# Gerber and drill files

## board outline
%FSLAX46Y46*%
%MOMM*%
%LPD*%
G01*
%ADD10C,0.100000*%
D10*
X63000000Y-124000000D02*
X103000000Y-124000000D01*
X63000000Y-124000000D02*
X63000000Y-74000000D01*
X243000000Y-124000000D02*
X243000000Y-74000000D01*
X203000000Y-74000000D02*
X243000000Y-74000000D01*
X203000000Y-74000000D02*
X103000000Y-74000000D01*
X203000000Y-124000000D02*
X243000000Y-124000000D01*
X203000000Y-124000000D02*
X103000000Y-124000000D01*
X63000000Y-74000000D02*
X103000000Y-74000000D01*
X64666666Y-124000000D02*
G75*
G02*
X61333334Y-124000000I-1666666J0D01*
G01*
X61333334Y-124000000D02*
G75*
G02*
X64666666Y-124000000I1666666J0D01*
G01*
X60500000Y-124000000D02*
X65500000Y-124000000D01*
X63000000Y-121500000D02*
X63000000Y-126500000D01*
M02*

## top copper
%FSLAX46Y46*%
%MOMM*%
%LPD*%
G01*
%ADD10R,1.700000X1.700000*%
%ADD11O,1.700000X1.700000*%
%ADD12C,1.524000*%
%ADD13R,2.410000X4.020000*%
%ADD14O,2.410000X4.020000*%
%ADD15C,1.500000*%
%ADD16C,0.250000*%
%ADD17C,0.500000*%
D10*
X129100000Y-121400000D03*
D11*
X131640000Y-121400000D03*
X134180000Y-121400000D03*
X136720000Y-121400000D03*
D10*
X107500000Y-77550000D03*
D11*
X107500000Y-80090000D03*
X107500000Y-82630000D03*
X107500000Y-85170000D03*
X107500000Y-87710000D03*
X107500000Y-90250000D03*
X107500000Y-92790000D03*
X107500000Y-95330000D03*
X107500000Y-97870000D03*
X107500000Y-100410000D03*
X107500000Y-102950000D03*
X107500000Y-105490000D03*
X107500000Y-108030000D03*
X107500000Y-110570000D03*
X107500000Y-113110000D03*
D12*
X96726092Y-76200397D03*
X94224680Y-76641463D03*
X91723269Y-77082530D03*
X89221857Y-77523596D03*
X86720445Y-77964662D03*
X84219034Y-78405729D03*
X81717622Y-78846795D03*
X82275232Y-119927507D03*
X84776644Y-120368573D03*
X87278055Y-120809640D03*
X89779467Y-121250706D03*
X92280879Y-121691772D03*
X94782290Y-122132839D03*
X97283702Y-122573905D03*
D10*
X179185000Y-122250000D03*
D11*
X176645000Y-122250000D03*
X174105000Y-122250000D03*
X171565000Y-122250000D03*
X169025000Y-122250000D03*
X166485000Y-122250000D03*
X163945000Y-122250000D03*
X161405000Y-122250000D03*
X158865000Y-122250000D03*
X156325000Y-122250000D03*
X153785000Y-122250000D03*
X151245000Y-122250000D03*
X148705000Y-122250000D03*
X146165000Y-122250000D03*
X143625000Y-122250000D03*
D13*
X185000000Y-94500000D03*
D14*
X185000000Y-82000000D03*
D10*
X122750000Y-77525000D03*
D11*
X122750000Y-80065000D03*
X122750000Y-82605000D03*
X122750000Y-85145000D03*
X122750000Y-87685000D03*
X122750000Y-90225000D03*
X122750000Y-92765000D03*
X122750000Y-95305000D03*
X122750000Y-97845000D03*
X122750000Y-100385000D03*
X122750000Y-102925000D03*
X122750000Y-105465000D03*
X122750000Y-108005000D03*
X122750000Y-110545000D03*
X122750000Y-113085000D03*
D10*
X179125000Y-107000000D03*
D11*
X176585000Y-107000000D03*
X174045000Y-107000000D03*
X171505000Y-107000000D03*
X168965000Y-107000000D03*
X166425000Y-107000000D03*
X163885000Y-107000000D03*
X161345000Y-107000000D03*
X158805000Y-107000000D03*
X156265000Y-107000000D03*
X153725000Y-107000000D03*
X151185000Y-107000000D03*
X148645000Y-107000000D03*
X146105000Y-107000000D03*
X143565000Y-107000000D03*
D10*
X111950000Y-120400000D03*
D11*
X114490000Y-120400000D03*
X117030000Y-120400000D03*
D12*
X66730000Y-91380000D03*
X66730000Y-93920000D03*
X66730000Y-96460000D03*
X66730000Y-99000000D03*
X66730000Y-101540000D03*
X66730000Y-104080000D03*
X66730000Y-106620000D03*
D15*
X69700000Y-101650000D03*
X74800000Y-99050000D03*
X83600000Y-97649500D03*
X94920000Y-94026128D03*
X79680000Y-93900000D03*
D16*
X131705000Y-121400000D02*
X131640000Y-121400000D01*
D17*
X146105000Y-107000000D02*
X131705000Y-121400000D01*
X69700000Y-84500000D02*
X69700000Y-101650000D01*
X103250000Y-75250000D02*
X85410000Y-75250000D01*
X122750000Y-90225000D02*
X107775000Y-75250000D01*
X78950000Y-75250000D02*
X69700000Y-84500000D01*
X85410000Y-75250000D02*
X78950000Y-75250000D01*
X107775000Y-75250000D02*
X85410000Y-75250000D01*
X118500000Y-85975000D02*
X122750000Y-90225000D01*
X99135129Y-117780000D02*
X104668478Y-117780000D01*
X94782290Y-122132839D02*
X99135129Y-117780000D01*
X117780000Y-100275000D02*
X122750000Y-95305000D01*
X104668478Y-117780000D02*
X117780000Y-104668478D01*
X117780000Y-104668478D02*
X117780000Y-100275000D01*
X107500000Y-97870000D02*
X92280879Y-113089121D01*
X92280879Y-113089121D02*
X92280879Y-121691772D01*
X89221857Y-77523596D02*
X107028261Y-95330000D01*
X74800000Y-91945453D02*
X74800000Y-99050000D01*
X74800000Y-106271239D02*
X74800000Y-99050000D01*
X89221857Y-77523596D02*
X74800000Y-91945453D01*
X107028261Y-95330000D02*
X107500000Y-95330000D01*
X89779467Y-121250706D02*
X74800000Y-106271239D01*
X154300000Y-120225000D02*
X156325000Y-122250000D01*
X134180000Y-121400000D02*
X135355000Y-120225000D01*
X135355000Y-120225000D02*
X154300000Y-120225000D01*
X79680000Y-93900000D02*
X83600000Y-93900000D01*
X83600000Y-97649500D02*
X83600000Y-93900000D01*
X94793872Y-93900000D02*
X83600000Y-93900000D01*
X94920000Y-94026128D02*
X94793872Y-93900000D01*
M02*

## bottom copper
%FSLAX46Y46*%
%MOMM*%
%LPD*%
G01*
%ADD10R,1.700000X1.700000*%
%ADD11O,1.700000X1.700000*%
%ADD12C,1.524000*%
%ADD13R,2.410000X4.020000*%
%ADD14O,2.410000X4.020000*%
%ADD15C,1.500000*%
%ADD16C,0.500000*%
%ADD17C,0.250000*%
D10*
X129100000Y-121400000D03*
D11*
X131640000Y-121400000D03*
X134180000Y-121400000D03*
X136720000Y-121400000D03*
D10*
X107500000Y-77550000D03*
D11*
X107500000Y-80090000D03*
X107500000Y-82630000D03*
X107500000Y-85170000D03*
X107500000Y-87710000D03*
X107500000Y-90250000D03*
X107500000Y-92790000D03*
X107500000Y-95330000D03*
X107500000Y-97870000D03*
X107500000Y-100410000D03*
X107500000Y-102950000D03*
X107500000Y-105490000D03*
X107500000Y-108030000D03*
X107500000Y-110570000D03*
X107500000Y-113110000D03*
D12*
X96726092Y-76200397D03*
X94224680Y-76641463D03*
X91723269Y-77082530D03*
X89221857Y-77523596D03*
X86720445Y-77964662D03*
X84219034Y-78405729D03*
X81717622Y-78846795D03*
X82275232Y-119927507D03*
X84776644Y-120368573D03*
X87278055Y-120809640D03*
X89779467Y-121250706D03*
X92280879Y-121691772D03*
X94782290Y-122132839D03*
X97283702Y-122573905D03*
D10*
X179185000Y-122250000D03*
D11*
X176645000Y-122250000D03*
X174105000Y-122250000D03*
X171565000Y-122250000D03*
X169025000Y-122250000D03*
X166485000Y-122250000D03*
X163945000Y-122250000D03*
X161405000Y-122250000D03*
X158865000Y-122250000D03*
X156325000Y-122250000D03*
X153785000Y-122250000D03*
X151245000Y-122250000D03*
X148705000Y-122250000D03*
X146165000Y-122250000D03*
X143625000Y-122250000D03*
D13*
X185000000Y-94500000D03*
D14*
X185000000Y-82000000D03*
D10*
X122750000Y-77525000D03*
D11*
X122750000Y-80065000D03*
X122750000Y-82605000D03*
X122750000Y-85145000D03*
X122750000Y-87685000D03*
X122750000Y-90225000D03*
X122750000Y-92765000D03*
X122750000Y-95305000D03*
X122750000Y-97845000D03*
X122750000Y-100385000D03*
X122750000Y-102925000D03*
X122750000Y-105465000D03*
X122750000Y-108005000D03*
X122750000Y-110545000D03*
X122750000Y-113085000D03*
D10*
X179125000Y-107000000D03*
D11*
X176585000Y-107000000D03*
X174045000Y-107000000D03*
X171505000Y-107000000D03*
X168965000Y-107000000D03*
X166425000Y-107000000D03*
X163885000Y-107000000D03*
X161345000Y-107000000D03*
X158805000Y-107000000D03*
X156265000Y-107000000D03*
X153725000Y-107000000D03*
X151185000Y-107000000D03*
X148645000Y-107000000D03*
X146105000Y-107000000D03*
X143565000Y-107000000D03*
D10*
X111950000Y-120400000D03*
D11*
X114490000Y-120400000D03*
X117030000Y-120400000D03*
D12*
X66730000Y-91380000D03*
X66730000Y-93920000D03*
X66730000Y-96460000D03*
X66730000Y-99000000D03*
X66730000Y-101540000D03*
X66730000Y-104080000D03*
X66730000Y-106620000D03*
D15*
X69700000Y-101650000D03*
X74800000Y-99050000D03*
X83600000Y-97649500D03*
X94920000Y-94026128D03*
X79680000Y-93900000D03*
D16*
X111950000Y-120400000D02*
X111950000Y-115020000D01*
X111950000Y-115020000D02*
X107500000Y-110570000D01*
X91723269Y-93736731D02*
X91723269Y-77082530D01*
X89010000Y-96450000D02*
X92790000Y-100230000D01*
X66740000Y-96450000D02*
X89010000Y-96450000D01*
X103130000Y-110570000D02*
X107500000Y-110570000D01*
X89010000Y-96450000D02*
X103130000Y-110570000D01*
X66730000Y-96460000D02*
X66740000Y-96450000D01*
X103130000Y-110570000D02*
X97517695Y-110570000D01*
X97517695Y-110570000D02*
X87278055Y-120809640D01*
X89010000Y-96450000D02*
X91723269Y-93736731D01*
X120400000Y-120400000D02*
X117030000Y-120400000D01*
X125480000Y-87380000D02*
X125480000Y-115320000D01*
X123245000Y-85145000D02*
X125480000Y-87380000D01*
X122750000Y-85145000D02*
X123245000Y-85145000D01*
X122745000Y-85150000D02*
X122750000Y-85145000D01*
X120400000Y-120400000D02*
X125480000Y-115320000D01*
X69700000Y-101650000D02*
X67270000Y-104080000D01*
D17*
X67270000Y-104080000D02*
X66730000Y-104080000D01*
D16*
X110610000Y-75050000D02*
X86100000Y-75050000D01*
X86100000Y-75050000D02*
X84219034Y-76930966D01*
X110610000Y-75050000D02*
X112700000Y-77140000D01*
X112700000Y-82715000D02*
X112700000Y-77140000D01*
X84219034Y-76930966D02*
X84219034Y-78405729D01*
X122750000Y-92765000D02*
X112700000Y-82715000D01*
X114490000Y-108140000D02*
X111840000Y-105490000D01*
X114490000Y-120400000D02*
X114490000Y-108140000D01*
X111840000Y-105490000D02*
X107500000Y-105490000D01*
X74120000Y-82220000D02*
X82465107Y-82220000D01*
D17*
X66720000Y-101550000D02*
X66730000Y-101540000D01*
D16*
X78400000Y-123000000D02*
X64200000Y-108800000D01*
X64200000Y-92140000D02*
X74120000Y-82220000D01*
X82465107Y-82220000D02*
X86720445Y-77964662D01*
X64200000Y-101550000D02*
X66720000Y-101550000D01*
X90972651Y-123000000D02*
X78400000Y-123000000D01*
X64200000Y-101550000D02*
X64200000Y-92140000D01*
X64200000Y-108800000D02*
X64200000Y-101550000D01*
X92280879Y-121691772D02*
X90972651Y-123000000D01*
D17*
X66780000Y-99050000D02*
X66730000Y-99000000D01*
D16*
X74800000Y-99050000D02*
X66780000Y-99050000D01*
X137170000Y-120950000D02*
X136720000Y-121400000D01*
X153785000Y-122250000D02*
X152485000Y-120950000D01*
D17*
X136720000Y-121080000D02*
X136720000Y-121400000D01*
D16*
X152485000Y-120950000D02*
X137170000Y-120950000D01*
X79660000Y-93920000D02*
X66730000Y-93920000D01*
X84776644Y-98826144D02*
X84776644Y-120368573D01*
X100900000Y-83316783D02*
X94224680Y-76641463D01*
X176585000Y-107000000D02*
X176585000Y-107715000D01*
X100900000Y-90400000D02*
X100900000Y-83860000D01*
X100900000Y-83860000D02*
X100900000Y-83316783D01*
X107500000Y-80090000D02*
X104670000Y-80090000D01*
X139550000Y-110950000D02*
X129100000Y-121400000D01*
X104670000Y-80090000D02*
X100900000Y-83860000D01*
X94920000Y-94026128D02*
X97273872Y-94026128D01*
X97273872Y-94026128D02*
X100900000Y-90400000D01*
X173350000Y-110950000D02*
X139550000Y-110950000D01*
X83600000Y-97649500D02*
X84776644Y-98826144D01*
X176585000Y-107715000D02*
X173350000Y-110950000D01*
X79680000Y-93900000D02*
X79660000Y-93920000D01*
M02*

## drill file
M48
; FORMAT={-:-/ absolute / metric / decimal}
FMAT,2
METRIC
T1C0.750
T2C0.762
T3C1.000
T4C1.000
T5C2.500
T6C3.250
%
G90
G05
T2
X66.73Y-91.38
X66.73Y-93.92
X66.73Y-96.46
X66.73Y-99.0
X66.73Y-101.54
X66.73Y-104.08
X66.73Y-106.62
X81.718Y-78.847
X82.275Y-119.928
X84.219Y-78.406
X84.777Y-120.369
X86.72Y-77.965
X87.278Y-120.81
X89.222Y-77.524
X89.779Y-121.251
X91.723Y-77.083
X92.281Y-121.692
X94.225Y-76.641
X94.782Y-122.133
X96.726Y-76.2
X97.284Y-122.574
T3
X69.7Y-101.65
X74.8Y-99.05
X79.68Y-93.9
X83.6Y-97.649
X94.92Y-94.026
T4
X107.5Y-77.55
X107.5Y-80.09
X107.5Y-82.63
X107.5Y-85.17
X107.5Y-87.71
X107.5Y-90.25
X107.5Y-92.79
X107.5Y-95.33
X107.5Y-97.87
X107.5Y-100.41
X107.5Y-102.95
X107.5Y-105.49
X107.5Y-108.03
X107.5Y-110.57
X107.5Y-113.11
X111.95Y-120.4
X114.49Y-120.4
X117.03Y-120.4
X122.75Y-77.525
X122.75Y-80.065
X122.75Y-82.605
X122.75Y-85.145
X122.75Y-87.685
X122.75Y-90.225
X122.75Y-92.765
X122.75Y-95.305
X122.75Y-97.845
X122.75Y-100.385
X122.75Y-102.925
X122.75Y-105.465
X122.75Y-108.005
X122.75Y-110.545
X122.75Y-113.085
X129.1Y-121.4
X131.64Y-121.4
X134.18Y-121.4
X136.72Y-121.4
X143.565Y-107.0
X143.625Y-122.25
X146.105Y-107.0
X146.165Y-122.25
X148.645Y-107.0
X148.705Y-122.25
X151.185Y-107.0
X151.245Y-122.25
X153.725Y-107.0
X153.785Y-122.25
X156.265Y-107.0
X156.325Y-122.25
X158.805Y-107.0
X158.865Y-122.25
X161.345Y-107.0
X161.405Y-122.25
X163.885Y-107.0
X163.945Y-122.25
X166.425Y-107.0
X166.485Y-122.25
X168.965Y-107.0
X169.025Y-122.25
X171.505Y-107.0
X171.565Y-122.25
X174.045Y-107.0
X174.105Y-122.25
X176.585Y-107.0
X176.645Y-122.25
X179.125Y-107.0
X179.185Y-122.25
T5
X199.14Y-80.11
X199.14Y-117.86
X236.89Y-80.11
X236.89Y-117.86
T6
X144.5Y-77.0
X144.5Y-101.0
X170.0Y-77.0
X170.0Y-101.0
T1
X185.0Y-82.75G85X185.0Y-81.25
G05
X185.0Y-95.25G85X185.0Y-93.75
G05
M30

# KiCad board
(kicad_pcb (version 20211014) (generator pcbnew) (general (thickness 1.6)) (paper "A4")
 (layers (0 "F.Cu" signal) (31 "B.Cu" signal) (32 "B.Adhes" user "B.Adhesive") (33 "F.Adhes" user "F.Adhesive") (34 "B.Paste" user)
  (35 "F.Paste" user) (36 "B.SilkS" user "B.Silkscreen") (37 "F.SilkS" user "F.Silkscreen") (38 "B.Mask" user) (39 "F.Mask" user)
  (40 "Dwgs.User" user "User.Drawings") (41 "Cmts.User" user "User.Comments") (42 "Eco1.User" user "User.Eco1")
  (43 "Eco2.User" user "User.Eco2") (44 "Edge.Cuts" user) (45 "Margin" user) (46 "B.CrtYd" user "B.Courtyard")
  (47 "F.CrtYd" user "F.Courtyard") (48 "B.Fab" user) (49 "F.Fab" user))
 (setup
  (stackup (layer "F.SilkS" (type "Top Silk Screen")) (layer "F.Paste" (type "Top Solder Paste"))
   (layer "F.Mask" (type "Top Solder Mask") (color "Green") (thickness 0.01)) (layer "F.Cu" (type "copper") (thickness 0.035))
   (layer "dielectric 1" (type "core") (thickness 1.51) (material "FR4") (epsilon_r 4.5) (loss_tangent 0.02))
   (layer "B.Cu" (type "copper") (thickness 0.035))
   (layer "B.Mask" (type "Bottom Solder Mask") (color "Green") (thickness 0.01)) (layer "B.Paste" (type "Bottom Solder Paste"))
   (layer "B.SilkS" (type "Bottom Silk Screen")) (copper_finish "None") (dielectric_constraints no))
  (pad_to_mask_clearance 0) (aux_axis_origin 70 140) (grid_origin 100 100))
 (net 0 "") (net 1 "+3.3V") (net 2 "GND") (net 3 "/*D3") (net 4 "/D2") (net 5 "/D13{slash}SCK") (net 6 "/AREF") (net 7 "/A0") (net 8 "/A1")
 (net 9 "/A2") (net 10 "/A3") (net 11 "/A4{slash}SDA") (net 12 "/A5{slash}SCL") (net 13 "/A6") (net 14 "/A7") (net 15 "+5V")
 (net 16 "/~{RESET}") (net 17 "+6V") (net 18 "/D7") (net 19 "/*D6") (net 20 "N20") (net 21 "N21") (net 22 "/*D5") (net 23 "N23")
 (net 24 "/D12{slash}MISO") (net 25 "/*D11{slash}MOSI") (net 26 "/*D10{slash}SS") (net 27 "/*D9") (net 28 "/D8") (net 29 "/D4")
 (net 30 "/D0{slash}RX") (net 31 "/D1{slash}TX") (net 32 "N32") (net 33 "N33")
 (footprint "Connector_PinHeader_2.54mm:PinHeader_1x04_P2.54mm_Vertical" (layer "F.Cu") (at 129.1 121.4 90)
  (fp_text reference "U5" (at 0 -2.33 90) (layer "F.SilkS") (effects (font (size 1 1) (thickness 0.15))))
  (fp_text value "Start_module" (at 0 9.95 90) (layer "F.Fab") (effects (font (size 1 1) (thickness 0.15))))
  (pad "1" thru_hole rect (at 0 0 90) (size 1.7 1.7) (drill 1) (layers *.Cu *.Mask) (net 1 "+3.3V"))
  (pad "2" thru_hole oval (at 0 2.54 90) (size 1.7 1.7) (drill 1) (layers *.Cu *.Mask) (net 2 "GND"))
  (pad "3" thru_hole oval (at 0 5.08 90) (size 1.7 1.7) (drill 1) (layers *.Cu *.Mask) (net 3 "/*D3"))
  (pad "4" thru_hole oval (at 0 7.62 90) (size 1.7 1.7) (drill 1) (layers *.Cu *.Mask) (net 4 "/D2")))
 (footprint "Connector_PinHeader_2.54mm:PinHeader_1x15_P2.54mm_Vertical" (layer "F.Cu") (at 107.5 77.55)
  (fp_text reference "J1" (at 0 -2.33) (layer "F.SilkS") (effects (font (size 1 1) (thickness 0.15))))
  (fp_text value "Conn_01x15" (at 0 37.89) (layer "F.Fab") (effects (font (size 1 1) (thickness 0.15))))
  (pad "1" thru_hole rect (at 0 0) (size 1.7 1.7) (drill 1) (layers *.Cu *.Mask) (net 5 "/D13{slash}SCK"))
  (pad "2" thru_hole oval (at 0 2.54) (size 1.7 1.7) (drill 1) (layers *.Cu *.Mask) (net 1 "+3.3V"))
  (pad "3" thru_hole oval (at 0 5.08) (size 1.7 1.7) (drill 1) (layers *.Cu *.Mask) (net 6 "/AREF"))
  (pad "4" thru_hole oval (at 0 7.62) (size 1.7 1.7) (drill 1) (layers *.Cu *.Mask) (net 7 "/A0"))
  (pad "5" thru_hole oval (at 0 10.16) (size 1.7 1.7) (drill 1) (layers *.Cu *.Mask) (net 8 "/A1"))
  (pad "6" thru_hole oval (at 0 12.7) (size 1.7 1.7) (drill 1) (layers *.Cu *.Mask) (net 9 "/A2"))
  (pad "7" thru_hole oval (at 0 15.24) (size 1.7 1.7) (drill 1) (layers *.Cu *.Mask) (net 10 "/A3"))
  (pad "8" thru_hole oval (at 0 17.78) (size 1.7 1.7) (drill 1) (layers *.Cu *.Mask) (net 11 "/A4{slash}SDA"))
  (pad "9" thru_hole oval (at 0 20.32) (size 1.7 1.7) (drill 1) (layers *.Cu *.Mask) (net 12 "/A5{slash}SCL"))
  (pad "10" thru_hole oval (at 0 22.86) (size 1.7 1.7) (drill 1) (layers *.Cu *.Mask) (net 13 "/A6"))
  (pad "11" thru_hole oval (at 0 25.4) (size 1.7 1.7) (drill 1) (layers *.Cu *.Mask) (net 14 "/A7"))
  (pad "12" thru_hole oval (at 0 27.94) (size 1.7 1.7) (drill 1) (layers *.Cu *.Mask) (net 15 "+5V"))
  (pad "13" thru_hole oval (at 0 30.48) (size 1.7 1.7) (drill 1) (layers *.Cu *.Mask) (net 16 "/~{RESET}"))
  (pad "14" thru_hole oval (at 0 33.02) (size 1.7 1.7) (drill 1) (layers *.Cu *.Mask) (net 2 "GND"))
  (pad "15" thru_hole oval (at 0 35.56) (size 1.7 1.7) (drill 1) (layers *.Cu *.Mask) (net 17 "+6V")))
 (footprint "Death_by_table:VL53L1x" (layer "F.Cu") (at 96.726092 76.200397 -170)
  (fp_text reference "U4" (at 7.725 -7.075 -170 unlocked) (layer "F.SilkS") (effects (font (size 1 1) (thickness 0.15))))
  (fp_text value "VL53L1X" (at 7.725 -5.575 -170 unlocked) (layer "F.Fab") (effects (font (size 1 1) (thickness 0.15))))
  (pad "1" thru_hole circle (at 0 0 190) (size 1.524 1.524) (drill 0.762) (layers *.Cu *.Mask) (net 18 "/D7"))
  (pad "2" thru_hole circle (at 2.54 0 190) (size 1.524 1.524) (drill 0.762) (layers *.Cu *.Mask) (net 1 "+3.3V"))
  (pad "3" thru_hole circle (at 5.08 0 190) (size 1.524 1.524) (drill 0.762) (layers *.Cu *.Mask) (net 2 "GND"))
  (pad "4" thru_hole circle (at 7.62 0 190) (size 1.524 1.524) (drill 0.762) (layers *.Cu *.Mask) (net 11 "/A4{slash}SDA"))
  (pad "5" thru_hole circle (at 10.16 0 190) (size 1.524 1.524) (drill 0.762) (layers *.Cu *.Mask) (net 12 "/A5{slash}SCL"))
  (pad "6" thru_hole circle (at 12.7 0 190) (size 1.524 1.524) (drill 0.762) (layers *.Cu *.Mask) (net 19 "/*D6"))
  (pad "7" thru_hole circle (at 15.24 0 190) (size 1.524 1.524) (drill 0.762) (layers *.Cu *.Mask) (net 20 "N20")))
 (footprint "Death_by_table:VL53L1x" (layer "F.Cu") (at 82.275232 119.927507 -10)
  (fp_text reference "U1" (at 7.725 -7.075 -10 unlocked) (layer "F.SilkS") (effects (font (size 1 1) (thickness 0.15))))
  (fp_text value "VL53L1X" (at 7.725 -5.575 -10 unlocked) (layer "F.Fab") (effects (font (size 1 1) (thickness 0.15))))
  (pad "1" thru_hole circle (at 0 0 350) (size 1.524 1.524) (drill 0.762) (layers *.Cu *.Mask) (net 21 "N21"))
  (pad "2" thru_hole circle (at 2.54 0 350) (size 1.524 1.524) (drill 0.762) (layers *.Cu *.Mask) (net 1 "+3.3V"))
  (pad "3" thru_hole circle (at 5.08 0 350) (size 1.524 1.524) (drill 0.762) (layers *.Cu *.Mask) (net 2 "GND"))
  (pad "4" thru_hole circle (at 7.62 0 350) (size 1.524 1.524) (drill 0.762) (layers *.Cu *.Mask) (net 11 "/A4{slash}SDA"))
  (pad "5" thru_hole circle (at 10.16 0 350) (size 1.524 1.524) (drill 0.762) (layers *.Cu *.Mask) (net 12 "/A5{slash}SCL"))
  (pad "6" thru_hole circle (at 12.7 0 350) (size 1.524 1.524) (drill 0.762) (layers *.Cu *.Mask) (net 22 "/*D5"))
  (pad "7" thru_hole circle (at 15.24 0 350) (size 1.524 1.524) (drill 0.762) (layers *.Cu *.Mask) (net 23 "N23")))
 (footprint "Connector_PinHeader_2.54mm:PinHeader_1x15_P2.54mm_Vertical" (layer "F.Cu") (at 179.185 122.25 -90)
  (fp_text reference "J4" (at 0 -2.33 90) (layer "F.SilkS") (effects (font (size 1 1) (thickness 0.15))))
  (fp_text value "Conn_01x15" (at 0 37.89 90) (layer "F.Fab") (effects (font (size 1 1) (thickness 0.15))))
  (pad "1" thru_hole rect (at 0 0 270) (size 1.7 1.7) (drill 1) (layers *.Cu *.Mask) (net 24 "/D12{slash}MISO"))
  (pad "2" thru_hole oval (at 0 2.54 270) (size 1.7 1.7) (drill 1) (layers *.Cu *.Mask) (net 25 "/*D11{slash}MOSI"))
  (pad "3" thru_hole oval (at 0 5.08 270) (size 1.7 1.7) (drill 1) (layers *.Cu *.Mask) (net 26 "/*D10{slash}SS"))
  (pad "4" thru_hole oval (at 0 7.62 270) (size 1.7 1.7) (drill 1) (layers *.Cu *.Mask) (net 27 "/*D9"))
  (pad "5" thru_hole oval (at 0 10.16 270) (size 1.7 1.7) (drill 1) (layers *.Cu *.Mask) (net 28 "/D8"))
  (pad "6" thru_hole oval (at 0 12.7 270) (size 1.7 1.7) (drill 1) (layers *.Cu *.Mask) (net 18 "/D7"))
  (pad "7" thru_hole oval (at 0 15.24 270) (size 1.7 1.7) (drill 1) (layers *.Cu *.Mask) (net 19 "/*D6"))
  (pad "8" thru_hole oval (at 0 17.78 270) (size 1.7 1.7) (drill 1) (layers *.Cu *.Mask) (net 22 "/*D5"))
  (pad "9" thru_hole oval (at 0 20.32 270) (size 1.7 1.7) (drill 1) (layers *.Cu *.Mask) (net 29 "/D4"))
  (pad "10" thru_hole oval (at 0 22.86 270) (size 1.7 1.7) (drill 1) (layers *.Cu *.Mask) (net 3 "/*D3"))
  (pad "11" thru_hole oval (at 0 25.4 270) (size 1.7 1.7) (drill 1) (layers *.Cu *.Mask) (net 4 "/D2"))
  (pad "12" thru_hole oval (at 0 27.94 270) (size 1.7 1.7) (drill 1) (layers *.Cu *.Mask) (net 2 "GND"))
  (pad "13" thru_hole oval (at 0 30.48 270) (size 1.7 1.7) (drill 1) (layers *.Cu *.Mask) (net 16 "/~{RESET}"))
  (pad "14" thru_hole oval (at 0 33.02 270) (size 1.7 1.7) (drill 1) (layers *.Cu *.Mask) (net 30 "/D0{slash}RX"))
  (pad "15" thru_hole oval (at 0 35.56 270) (size 1.7 1.7) (drill 1) (layers *.Cu *.Mask) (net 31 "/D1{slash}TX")))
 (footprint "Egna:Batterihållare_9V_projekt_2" (layer "F.Cu") (at 185 74 180)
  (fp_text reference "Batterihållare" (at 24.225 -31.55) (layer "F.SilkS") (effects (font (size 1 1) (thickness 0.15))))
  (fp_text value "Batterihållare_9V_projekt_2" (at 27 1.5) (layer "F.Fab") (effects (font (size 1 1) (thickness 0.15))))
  (pad "" np_thru_hole circle (at 15 -27 180) (size 2.3 2.3) (drill 3.25) (layers F&B.Cu *.Mask))
  (pad "" np_thru_hole circle (at 40.5 -3 180) (size 2.3 2.3) (drill 3.25) (layers F&B.Cu *.Mask))
  (pad "" np_thru_hole circle (at 15 -3 180) (size 2.3 2.3) (drill 3.25) (layers F&B.Cu *.Mask))
  (pad "" np_thru_hole circle (at 40.5 -27 180) (size 2.3 2.3) (drill 3.25) (layers F&B.Cu *.Mask))
  (pad "1" thru_hole rect (at 0 -20.5 180) (size 2.41 4.02) (drill oval 0.75 2.25) (layers *.Cu *.Mask))
  (pad "2" thru_hole oval (at 0 -8 180) (size 2.41 4.02) (drill oval 0.75 2.25) (layers *.Cu *.Mask)))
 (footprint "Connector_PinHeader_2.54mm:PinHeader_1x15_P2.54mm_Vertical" (layer "F.Cu") (at 122.75 77.525)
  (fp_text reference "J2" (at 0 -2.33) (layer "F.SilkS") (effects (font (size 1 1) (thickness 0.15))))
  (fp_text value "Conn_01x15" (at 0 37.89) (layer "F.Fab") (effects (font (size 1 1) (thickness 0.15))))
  (pad "1" thru_hole rect (at 0 0) (size 1.7 1.7) (drill 1) (layers *.Cu *.Mask) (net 24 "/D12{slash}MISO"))
  (pad "2" thru_hole oval (at 0 2.54) (size 1.7 1.7) (drill 1) (layers *.Cu *.Mask) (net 25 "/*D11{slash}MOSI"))
  (pad "3" thru_hole oval (at 0 5.08) (size 1.7 1.7) (drill 1) (layers *.Cu *.Mask) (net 26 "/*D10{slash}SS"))
  (pad "4" thru_hole oval (at 0 7.62) (size 1.7 1.7) (drill 1) (layers *.Cu *.Mask) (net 27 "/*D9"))
  (pad "5" thru_hole oval (at 0 10.16) (size 1.7 1.7) (drill 1) (layers *.Cu *.Mask) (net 28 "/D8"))
  (pad "6" thru_hole oval (at 0 12.7) (size 1.7 1.7) (drill 1) (layers *.Cu *.Mask) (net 18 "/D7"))
  (pad "7" thru_hole oval (at 0 15.24) (size 1.7 1.7) (drill 1) (layers *.Cu *.Mask) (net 19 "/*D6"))
  (pad "8" thru_hole oval (at 0 17.78) (size 1.7 1.7) (drill 1) (layers *.Cu *.Mask) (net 22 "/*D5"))
  (pad "9" thru_hole oval (at 0 20.32) (size 1.7 1.7) (drill 1) (layers *.Cu *.Mask) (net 29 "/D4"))
  (pad "10" thru_hole oval (at 0 22.86) (size 1.7 1.7) (drill 1) (layers *.Cu *.Mask) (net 3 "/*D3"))
  (pad "11" thru_hole oval (at 0 25.4) (size 1.7 1.7) (drill 1) (layers *.Cu *.Mask) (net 4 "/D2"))
  (pad "12" thru_hole oval (at 0 27.94) (size 1.7 1.7) (drill 1) (layers *.Cu *.Mask) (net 2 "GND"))
  (pad "13" thru_hole oval (at 0 30.48) (size 1.7 1.7) (drill 1) (layers *.Cu *.Mask) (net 16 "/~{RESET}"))
  (pad "14" thru_hole oval (at 0 33.02) (size 1.7 1.7) (drill 1) (layers *.Cu *.Mask) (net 30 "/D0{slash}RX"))
  (pad "15" thru_hole oval (at 0 35.56) (size 1.7 1.7) (drill 1) (layers *.Cu *.Mask) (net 31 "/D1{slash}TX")))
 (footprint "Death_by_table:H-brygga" (layer "F.Cu") (at 195.14 121.86)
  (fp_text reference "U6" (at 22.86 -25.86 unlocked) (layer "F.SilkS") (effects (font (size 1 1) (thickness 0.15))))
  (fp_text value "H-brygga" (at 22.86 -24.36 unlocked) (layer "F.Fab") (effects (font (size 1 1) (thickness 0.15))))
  (pad "" np_thru_hole circle (at 4 -4) (size 2.5 2.5) (drill 2.5) (layers F&B.Cu *.Mask))
  (pad "" np_thru_hole circle (at 41.75 -41.75) (size 2.5 2.5) (drill 2.5) (layers F&B.Cu *.Mask))
  (pad "" np_thru_hole circle (at 4 -41.75) (size 2.5 2.5) (drill 2.5) (layers F&B.Cu *.Mask))
  (pad "" np_thru_hole circle (at 41.75 -4) (size 2.5 2.5) (drill 2.5) (layers F&B.Cu *.Mask)))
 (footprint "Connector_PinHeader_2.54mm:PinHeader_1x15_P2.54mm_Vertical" (layer "F.Cu") (at 179.125 107 -90)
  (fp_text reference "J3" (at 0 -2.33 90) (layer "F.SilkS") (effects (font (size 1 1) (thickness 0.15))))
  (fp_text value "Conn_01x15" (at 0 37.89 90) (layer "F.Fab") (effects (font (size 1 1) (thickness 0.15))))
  (pad "1" thru_hole rect (at 0 0 270) (size 1.7 1.7) (drill 1) (layers *.Cu *.Mask) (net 5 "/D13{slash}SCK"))
  (pad "2" thru_hole oval (at 0 2.54 270) (size 1.7 1.7) (drill 1) (layers *.Cu *.Mask) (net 1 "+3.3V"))
  (pad "3" thru_hole oval (at 0 5.08 270) (size 1.7 1.7) (drill 1) (layers *.Cu *.Mask) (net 6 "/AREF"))
  (pad "4" thru_hole oval (at 0 7.62 270) (size 1.7 1.7) (drill 1) (layers *.Cu *.Mask) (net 7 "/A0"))
  (pad "5" thru_hole oval (at 0 10.16 270) (size 1.7 1.7) (drill 1) (layers *.Cu *.Mask) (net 8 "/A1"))
  (pad "6" thru_hole oval (at 0 12.7 270) (size 1.7 1.7) (drill 1) (layers *.Cu *.Mask) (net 9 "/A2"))
  (pad "7" thru_hole oval (at 0 15.24 270) (size 1.7 1.7) (drill 1) (layers *.Cu *.Mask) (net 10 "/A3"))
  (pad "8" thru_hole oval (at 0 17.78 270) (size 1.7 1.7) (drill 1) (layers *.Cu *.Mask) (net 11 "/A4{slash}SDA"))
  (pad "9" thru_hole oval (at 0 20.32 270) (size 1.7 1.7) (drill 1) (layers *.Cu *.Mask) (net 12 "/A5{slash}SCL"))
  (pad "10" thru_hole oval (at 0 22.86 270) (size 1.7 1.7) (drill 1) (layers *.Cu *.Mask) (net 13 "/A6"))
  (pad "11" thru_hole oval (at 0 25.4 270) (size 1.7 1.7) (drill 1) (layers *.Cu *.Mask) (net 14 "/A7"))
  (pad "12" thru_hole oval (at 0 27.94 270) (size 1.7 1.7) (drill 1) (layers *.Cu *.Mask) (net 15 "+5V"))
  (pad "13" thru_hole oval (at 0 30.48 270) (size 1.7 1.7) (drill 1) (layers *.Cu *.Mask) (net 16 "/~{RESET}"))
  (pad "14" thru_hole oval (at 0 33.02 270) (size 1.7 1.7) (drill 1) (layers *.Cu *.Mask) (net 2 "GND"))
  (pad "15" thru_hole oval (at 0 35.56 270) (size 1.7 1.7) (drill 1) (layers *.Cu *.Mask) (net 17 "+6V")))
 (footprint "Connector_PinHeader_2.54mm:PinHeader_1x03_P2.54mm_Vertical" (layer "F.Cu") (at 111.95 120.4 90)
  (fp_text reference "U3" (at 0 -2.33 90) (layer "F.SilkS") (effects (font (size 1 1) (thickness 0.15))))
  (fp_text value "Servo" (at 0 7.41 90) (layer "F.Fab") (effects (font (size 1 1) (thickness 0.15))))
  (pad "1" thru_hole rect (at 0 0 90) (size 1.7 1.7) (drill 1) (layers *.Cu *.Mask) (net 2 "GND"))
  (pad "2" thru_hole oval (at 0 2.54 90) (size 1.7 1.7) (drill 1) (layers *.Cu *.Mask) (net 15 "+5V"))
  (pad "3" thru_hole oval (at 0 5.08 90) (size 1.7 1.7) (drill 1) (layers *.Cu *.Mask) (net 27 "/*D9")))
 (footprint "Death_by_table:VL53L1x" (layer "F.Cu") (at 66.73 91.38 -90)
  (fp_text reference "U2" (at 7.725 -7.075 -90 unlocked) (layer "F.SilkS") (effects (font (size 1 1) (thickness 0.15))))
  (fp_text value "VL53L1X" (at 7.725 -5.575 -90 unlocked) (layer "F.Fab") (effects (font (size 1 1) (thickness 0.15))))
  (pad "1" thru_hole circle (at 0 0 270) (size 1.524 1.524) (drill 0.762) (layers *.Cu *.Mask) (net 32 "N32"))
  (pad "2" thru_hole circle (at 2.54 0 270) (size 1.524 1.524) (drill 0.762) (layers *.Cu *.Mask) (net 1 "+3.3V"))
  (pad "3" thru_hole circle (at 5.08 0 270) (size 1.524 1.524) (drill 0.762) (layers *.Cu *.Mask) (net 2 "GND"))
  (pad "4" thru_hole circle (at 7.62 0 270) (size 1.524 1.524) (drill 0.762) (layers *.Cu *.Mask) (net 11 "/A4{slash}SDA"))
  (pad "5" thru_hole circle (at 10.16 0 270) (size 1.524 1.524) (drill 0.762) (layers *.Cu *.Mask) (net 12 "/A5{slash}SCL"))
  (pad "6" thru_hole circle (at 12.7 0 270) (size 1.524 1.524) (drill 0.762) (layers *.Cu *.Mask) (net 18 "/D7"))
  (pad "7" thru_hole circle (at 15.24 0 270) (size 1.524 1.524) (drill 0.762) (layers *.Cu *.Mask) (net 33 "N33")))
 (gr_line (start 63 124) (end 103 124) (layer "Edge.Cuts") (width 0.1))
 (gr_line (start 63 124) (end 63 74) (layer "Edge.Cuts") (width 0.1))
 (gr_line (start 243 124) (end 243 74) (layer "Edge.Cuts") (width 0.1))
 (gr_line (start 203 74) (end 243 74) (layer "Edge.Cuts") (width 0.1))
 (gr_line (start 203 74) (end 103 74) (layer "Edge.Cuts") (width 0.1))
 (gr_line (start 203 124) (end 243 124) (layer "Edge.Cuts") (width 0.1))
 (gr_line (start 203 124) (end 103 124) (layer "Edge.Cuts") (width 0.1))
 (gr_line (start 63 74) (end 103 74) (layer "Edge.Cuts") (width 0.1))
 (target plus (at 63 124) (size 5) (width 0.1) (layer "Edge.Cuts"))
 (segment (start 131.705 121.4) (end 131.64 121.4) (width 0.25) (layer "F.Cu") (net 2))
 (segment (start 146.105 107) (end 131.705 121.4) (width 0.5) (layer "F.Cu") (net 2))
 (segment (start 111.95 120.4) (end 111.95 115.02) (width 0.5) (layer "B.Cu") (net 2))
 (segment (start 111.95 115.02) (end 107.5 110.57) (width 0.5) (layer "B.Cu") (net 2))
 (segment (start 91.723269 93.736731) (end 91.723269 77.08253) (width 0.5) (layer "B.Cu") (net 2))
 (segment (start 89.01 96.45) (end 92.79 100.23) (width 0.5) (layer "B.Cu") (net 2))
 (segment (start 66.74 96.45) (end 89.01 96.45) (width 0.5) (layer "B.Cu") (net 2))
 (segment (start 103.13 110.57) (end 107.5 110.57) (width 0.5) (layer "B.Cu") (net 2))
 (segment (start 89.01 96.45) (end 103.13 110.57) (width 0.5) (layer "B.Cu") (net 2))
 (segment (start 66.73 96.46) (end 66.74 96.45) (width 0.5) (layer "B.Cu") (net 2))
 (segment (start 103.13 110.57) (end 97.517695 110.57) (width 0.5) (layer "B.Cu") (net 2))
 (segment (start 97.517695 110.57) (end 87.278055 120.80964) (width 0.5) (layer "B.Cu") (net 2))
 (segment (start 89.01 96.45) (end 91.723269 93.736731) (width 0.5) (layer "B.Cu") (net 2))
 (segment (start 120.4 120.4) (end 117.03 120.4) (width 0.5) (layer "B.Cu") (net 27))
 (segment (start 125.48 87.38) (end 125.48 115.32) (width 0.5) (layer "B.Cu") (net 27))
 (segment (start 123.245 85.145) (end 125.48 87.38) (width 0.5) (layer "B.Cu") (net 27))
 (segment (start 122.75 85.145) (end 123.245 85.145) (width 0.5) (layer "B.Cu") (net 27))
 (segment (start 122.745 85.15) (end 122.75 85.145) (width 0.5) (layer "B.Cu") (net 27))
 (segment (start 120.4 120.4) (end 125.48 115.32) (width 0.5) (layer "B.Cu") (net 27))
 (segment (start 69.7 84.5) (end 69.7 101.65) (width 0.5) (layer "F.Cu") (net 18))
 (segment (start 103.25 75.25) (end 85.41 75.25) (width 0.5) (layer "F.Cu") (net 18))
 (segment (start 122.75 90.225) (end 107.775 75.25) (width 0.5) (layer "F.Cu") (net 18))
 (segment (start 78.95 75.25) (end 69.7 84.5) (width 0.5) (layer "F.Cu") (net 18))
 (segment (start 85.41 75.25) (end 78.95 75.25) (width 0.5) (layer "F.Cu") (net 18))
 (segment (start 107.775 75.25) (end 85.41 75.25) (width 0.5) (layer "F.Cu") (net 18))
 (segment (start 118.5 85.975) (end 122.75 90.225) (width 0.5) (layer "F.Cu") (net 18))
 (via (at 69.7 101.65) (size 1.5) (drill 1) (layers "F.Cu" "B.Cu") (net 18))
 (segment (start 69.7 101.65) (end 67.27 104.08) (width 0.5) (layer "B.Cu") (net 18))
 (segment (start 67.27 104.08) (end 66.73 104.08) (width 0.25) (layer "B.Cu") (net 18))
 (segment (start 110.61 75.05) (end 86.1 75.05) (width 0.5) (layer "B.Cu") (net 19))
 (segment (start 86.1 75.05) (end 84.219034 76.930966) (width 0.5) (layer "B.Cu") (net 19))
 (segment (start 110.61 75.05) (end 112.7 77.14) (width 0.5) (layer "B.Cu") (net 19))
 (segment (start 112.7 82.715) (end 112.7 77.14) (width 0.5) (layer "B.Cu") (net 19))
 (segment (start 84.219034 76.930966) (end 84.219034 78.405729) (width 0.5) (layer "B.Cu") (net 19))
 (segment (start 122.75 92.765) (end 112.7 82.715) (width 0.5) (layer "B.Cu") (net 19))
 (segment (start 99.135129 117.78) (end 104.668478 117.78) (width 0.5) (layer "F.Cu") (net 22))
 (segment (start 94.78229 122.132839) (end 99.135129 117.78) (width 0.5) (layer "F.Cu") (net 22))
 (segment (start 117.78 100.275) (end 122.75 95.305) (width 0.5) (layer "F.Cu") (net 22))
 (segment (start 104.668478 117.78) (end 117.78 104.668478) (width 0.5) (layer "F.Cu") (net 22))
 (segment (start 117.78 104.668478) (end 117.78 100.275) (width 0.5) (layer "F.Cu") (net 22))
 (segment (start 114.49 108.14) (end 111.84 105.49) (width 0.5) (layer "B.Cu") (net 15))
 (segment (start 114.49 120.4) (end 114.49 108.14) (width 0.5) (layer "B.Cu") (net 15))
 (segment (start 111.84 105.49) (end 107.5 105.49) (width 0.5) (layer "B.Cu") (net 15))
 (segment (start 107.5 97.87) (end 92.280879 113.089121) (width 0.5) (layer "F.Cu") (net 12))
 (segment (start 92.280879 113.089121) (end 92.280879 121.691772) (width 0.5) (layer "F.Cu") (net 12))
 (segment (start 74.12 82.22) (end 82.465107 82.22) (width 0.5) (layer "B.Cu") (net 12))
 (segment (start 66.72 101.55) (end 66.73 101.54) (width 0.25) (layer "B.Cu") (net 12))
 (segment (start 78.4 123) (end 64.2 108.8) (width 0.5) (layer "B.Cu") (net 12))
 (segment (start 64.2 92.14) (end 74.12 82.22) (width 0.5) (layer "B.Cu") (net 12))
 (segment (start 82.465107 82.22) (end 86.720445 77.964662) (width 0.5) (layer "B.Cu") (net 12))
 (segment (start 64.2 101.55) (end 66.72 101.55) (width 0.5) (layer "B.Cu") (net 12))
 (segment (start 90.972651 123) (end 78.4 123) (width 0.5) (layer "B.Cu") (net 12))
 (segment (start 64.2 101.55) (end 64.2 92.14) (width 0.5) (layer "B.Cu") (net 12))
 (segment (start 64.2 108.8) (end 64.2 101.55) (width 0.5) (layer "B.Cu") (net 12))
 (segment (start 92.280879 121.691772) (end 90.972651 123) (width 0.5) (layer "B.Cu") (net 12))
 (segment (start 89.221857 77.523596) (end 107.028261 95.33) (width 0.5) (layer "F.Cu") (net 11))
 (segment (start 74.8 91.945453) (end 74.8 99.05) (width 0.5) (layer "F.Cu") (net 11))
 (segment (start 74.8 106.271239) (end 74.8 99.05) (width 0.5) (layer "F.Cu") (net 11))
 (segment (start 89.221857 77.523596) (end 74.8 91.945453) (width 0.5) (layer "F.Cu") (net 11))
 (segment (start 107.028261 95.33) (end 107.5 95.33) (width 0.5) (layer "F.Cu") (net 11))
 (segment (start 89.779467 121.250706) (end 74.8 106.271239) (width 0.5) (layer "F.Cu") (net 11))
 (via (at 74.8 99.05) (size 1.5) (drill 1) (layers "F.Cu" "B.Cu") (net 11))
 (segment (start 66.78 99.05) (end 66.73 99) (width 0.25) (layer "B.Cu") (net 11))
 (segment (start 74.8 99.05) (end 66.78 99.05) (width 0.5) (layer "B.Cu") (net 11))
 (segment (start 137.17 120.95) (end 136.72 121.4) (width 0.5) (layer "B.Cu") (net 4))
 (segment (start 153.785 122.25) (end 152.485 120.95) (width 0.5) (layer "B.Cu") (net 4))
 (segment (start 136.72 121.08) (end 136.72 121.4) (width 0.25) (layer "B.Cu") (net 4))
 (segment (start 152.485 120.95) (end 137.17 120.95) (width 0.5) (layer "B.Cu") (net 4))
 (segment (start 154.3 120.225) (end 156.325 122.25) (width 0.5) (layer "F.Cu") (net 3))
 (segment (start 134.18 121.4) (end 135.355 120.225) (width 0.5) (layer "F.Cu") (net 3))
 (segment (start 135.355 120.225) (end 154.3 120.225) (width 0.5) (layer "F.Cu") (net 3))
 (segment (start 79.68 93.9) (end 83.6 93.9) (width 0.5) (layer "F.Cu") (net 1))
 (segment (start 83.6 97.6495) (end 83.6 93.9) (width 0.5) (layer "F.Cu") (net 1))
 (segment (start 94.793872 93.9) (end 83.6 93.9) (width 0.5) (layer "F.Cu") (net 1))
 (segment (start 94.92 94.026128) (end 94.793872 93.9) (width 0.5) (layer "F.Cu") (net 1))
 (via (at 83.6 97.6495) (size 1.5) (drill 1) (layers "F.Cu" "B.Cu") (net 1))
 (via (at 94.92 94.026128) (size 1.5) (drill 1) (layers "F.Cu" "B.Cu") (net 1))
 (via (at 79.68 93.9) (size 1.5) (drill 1) (layers "F.Cu" "B.Cu") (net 1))
 (segment (start 79.66 93.92) (end 66.73 93.92) (width 0.5) (layer "B.Cu") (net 1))
 (segment (start 84.776644 98.826144) (end 84.776644 120.368573) (width 0.5) (layer "B.Cu") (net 1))
 (segment (start 100.9 83.316783) (end 94.22468 76.641463) (width 0.5) (layer "B.Cu") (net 1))
 (segment (start 176.585 107) (end 176.585 107.715) (width 0.5) (layer "B.Cu") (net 1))
 (segment (start 100.9 90.4) (end 100.9 83.86) (width 0.5) (layer "B.Cu") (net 1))
 (segment (start 100.9 83.86) (end 100.9 83.316783) (width 0.5) (layer "B.Cu") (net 1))
 (segment (start 107.5 80.09) (end 104.67 80.09) (width 0.5) (layer "B.Cu") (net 1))
 (segment (start 139.55 110.95) (end 129.1 121.4) (width 0.5) (layer "B.Cu") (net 1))
 (segment (start 104.67 80.09) (end 100.9 83.86) (width 0.5) (layer "B.Cu") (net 1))
 (segment (start 94.92 94.026128) (end 97.273872 94.026128) (width 0.5) (layer "B.Cu") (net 1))
 (segment (start 97.273872 94.026128) (end 100.9 90.4) (width 0.5) (layer "B.Cu") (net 1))
 (segment (start 173.35 110.95) (end 139.55 110.95) (width 0.5) (layer "B.Cu") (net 1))
 (segment (start 83.6 97.6495) (end 84.776644 98.826144) (width 0.5) (layer "B.Cu") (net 1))
 (segment (start 176.585 107.715) (end 173.35 110.95) (width 0.5) (layer "B.Cu") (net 1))
 (segment (start 79.68 93.9) (end 79.66 93.92) (width 0.5) (layer "B.Cu") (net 1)))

